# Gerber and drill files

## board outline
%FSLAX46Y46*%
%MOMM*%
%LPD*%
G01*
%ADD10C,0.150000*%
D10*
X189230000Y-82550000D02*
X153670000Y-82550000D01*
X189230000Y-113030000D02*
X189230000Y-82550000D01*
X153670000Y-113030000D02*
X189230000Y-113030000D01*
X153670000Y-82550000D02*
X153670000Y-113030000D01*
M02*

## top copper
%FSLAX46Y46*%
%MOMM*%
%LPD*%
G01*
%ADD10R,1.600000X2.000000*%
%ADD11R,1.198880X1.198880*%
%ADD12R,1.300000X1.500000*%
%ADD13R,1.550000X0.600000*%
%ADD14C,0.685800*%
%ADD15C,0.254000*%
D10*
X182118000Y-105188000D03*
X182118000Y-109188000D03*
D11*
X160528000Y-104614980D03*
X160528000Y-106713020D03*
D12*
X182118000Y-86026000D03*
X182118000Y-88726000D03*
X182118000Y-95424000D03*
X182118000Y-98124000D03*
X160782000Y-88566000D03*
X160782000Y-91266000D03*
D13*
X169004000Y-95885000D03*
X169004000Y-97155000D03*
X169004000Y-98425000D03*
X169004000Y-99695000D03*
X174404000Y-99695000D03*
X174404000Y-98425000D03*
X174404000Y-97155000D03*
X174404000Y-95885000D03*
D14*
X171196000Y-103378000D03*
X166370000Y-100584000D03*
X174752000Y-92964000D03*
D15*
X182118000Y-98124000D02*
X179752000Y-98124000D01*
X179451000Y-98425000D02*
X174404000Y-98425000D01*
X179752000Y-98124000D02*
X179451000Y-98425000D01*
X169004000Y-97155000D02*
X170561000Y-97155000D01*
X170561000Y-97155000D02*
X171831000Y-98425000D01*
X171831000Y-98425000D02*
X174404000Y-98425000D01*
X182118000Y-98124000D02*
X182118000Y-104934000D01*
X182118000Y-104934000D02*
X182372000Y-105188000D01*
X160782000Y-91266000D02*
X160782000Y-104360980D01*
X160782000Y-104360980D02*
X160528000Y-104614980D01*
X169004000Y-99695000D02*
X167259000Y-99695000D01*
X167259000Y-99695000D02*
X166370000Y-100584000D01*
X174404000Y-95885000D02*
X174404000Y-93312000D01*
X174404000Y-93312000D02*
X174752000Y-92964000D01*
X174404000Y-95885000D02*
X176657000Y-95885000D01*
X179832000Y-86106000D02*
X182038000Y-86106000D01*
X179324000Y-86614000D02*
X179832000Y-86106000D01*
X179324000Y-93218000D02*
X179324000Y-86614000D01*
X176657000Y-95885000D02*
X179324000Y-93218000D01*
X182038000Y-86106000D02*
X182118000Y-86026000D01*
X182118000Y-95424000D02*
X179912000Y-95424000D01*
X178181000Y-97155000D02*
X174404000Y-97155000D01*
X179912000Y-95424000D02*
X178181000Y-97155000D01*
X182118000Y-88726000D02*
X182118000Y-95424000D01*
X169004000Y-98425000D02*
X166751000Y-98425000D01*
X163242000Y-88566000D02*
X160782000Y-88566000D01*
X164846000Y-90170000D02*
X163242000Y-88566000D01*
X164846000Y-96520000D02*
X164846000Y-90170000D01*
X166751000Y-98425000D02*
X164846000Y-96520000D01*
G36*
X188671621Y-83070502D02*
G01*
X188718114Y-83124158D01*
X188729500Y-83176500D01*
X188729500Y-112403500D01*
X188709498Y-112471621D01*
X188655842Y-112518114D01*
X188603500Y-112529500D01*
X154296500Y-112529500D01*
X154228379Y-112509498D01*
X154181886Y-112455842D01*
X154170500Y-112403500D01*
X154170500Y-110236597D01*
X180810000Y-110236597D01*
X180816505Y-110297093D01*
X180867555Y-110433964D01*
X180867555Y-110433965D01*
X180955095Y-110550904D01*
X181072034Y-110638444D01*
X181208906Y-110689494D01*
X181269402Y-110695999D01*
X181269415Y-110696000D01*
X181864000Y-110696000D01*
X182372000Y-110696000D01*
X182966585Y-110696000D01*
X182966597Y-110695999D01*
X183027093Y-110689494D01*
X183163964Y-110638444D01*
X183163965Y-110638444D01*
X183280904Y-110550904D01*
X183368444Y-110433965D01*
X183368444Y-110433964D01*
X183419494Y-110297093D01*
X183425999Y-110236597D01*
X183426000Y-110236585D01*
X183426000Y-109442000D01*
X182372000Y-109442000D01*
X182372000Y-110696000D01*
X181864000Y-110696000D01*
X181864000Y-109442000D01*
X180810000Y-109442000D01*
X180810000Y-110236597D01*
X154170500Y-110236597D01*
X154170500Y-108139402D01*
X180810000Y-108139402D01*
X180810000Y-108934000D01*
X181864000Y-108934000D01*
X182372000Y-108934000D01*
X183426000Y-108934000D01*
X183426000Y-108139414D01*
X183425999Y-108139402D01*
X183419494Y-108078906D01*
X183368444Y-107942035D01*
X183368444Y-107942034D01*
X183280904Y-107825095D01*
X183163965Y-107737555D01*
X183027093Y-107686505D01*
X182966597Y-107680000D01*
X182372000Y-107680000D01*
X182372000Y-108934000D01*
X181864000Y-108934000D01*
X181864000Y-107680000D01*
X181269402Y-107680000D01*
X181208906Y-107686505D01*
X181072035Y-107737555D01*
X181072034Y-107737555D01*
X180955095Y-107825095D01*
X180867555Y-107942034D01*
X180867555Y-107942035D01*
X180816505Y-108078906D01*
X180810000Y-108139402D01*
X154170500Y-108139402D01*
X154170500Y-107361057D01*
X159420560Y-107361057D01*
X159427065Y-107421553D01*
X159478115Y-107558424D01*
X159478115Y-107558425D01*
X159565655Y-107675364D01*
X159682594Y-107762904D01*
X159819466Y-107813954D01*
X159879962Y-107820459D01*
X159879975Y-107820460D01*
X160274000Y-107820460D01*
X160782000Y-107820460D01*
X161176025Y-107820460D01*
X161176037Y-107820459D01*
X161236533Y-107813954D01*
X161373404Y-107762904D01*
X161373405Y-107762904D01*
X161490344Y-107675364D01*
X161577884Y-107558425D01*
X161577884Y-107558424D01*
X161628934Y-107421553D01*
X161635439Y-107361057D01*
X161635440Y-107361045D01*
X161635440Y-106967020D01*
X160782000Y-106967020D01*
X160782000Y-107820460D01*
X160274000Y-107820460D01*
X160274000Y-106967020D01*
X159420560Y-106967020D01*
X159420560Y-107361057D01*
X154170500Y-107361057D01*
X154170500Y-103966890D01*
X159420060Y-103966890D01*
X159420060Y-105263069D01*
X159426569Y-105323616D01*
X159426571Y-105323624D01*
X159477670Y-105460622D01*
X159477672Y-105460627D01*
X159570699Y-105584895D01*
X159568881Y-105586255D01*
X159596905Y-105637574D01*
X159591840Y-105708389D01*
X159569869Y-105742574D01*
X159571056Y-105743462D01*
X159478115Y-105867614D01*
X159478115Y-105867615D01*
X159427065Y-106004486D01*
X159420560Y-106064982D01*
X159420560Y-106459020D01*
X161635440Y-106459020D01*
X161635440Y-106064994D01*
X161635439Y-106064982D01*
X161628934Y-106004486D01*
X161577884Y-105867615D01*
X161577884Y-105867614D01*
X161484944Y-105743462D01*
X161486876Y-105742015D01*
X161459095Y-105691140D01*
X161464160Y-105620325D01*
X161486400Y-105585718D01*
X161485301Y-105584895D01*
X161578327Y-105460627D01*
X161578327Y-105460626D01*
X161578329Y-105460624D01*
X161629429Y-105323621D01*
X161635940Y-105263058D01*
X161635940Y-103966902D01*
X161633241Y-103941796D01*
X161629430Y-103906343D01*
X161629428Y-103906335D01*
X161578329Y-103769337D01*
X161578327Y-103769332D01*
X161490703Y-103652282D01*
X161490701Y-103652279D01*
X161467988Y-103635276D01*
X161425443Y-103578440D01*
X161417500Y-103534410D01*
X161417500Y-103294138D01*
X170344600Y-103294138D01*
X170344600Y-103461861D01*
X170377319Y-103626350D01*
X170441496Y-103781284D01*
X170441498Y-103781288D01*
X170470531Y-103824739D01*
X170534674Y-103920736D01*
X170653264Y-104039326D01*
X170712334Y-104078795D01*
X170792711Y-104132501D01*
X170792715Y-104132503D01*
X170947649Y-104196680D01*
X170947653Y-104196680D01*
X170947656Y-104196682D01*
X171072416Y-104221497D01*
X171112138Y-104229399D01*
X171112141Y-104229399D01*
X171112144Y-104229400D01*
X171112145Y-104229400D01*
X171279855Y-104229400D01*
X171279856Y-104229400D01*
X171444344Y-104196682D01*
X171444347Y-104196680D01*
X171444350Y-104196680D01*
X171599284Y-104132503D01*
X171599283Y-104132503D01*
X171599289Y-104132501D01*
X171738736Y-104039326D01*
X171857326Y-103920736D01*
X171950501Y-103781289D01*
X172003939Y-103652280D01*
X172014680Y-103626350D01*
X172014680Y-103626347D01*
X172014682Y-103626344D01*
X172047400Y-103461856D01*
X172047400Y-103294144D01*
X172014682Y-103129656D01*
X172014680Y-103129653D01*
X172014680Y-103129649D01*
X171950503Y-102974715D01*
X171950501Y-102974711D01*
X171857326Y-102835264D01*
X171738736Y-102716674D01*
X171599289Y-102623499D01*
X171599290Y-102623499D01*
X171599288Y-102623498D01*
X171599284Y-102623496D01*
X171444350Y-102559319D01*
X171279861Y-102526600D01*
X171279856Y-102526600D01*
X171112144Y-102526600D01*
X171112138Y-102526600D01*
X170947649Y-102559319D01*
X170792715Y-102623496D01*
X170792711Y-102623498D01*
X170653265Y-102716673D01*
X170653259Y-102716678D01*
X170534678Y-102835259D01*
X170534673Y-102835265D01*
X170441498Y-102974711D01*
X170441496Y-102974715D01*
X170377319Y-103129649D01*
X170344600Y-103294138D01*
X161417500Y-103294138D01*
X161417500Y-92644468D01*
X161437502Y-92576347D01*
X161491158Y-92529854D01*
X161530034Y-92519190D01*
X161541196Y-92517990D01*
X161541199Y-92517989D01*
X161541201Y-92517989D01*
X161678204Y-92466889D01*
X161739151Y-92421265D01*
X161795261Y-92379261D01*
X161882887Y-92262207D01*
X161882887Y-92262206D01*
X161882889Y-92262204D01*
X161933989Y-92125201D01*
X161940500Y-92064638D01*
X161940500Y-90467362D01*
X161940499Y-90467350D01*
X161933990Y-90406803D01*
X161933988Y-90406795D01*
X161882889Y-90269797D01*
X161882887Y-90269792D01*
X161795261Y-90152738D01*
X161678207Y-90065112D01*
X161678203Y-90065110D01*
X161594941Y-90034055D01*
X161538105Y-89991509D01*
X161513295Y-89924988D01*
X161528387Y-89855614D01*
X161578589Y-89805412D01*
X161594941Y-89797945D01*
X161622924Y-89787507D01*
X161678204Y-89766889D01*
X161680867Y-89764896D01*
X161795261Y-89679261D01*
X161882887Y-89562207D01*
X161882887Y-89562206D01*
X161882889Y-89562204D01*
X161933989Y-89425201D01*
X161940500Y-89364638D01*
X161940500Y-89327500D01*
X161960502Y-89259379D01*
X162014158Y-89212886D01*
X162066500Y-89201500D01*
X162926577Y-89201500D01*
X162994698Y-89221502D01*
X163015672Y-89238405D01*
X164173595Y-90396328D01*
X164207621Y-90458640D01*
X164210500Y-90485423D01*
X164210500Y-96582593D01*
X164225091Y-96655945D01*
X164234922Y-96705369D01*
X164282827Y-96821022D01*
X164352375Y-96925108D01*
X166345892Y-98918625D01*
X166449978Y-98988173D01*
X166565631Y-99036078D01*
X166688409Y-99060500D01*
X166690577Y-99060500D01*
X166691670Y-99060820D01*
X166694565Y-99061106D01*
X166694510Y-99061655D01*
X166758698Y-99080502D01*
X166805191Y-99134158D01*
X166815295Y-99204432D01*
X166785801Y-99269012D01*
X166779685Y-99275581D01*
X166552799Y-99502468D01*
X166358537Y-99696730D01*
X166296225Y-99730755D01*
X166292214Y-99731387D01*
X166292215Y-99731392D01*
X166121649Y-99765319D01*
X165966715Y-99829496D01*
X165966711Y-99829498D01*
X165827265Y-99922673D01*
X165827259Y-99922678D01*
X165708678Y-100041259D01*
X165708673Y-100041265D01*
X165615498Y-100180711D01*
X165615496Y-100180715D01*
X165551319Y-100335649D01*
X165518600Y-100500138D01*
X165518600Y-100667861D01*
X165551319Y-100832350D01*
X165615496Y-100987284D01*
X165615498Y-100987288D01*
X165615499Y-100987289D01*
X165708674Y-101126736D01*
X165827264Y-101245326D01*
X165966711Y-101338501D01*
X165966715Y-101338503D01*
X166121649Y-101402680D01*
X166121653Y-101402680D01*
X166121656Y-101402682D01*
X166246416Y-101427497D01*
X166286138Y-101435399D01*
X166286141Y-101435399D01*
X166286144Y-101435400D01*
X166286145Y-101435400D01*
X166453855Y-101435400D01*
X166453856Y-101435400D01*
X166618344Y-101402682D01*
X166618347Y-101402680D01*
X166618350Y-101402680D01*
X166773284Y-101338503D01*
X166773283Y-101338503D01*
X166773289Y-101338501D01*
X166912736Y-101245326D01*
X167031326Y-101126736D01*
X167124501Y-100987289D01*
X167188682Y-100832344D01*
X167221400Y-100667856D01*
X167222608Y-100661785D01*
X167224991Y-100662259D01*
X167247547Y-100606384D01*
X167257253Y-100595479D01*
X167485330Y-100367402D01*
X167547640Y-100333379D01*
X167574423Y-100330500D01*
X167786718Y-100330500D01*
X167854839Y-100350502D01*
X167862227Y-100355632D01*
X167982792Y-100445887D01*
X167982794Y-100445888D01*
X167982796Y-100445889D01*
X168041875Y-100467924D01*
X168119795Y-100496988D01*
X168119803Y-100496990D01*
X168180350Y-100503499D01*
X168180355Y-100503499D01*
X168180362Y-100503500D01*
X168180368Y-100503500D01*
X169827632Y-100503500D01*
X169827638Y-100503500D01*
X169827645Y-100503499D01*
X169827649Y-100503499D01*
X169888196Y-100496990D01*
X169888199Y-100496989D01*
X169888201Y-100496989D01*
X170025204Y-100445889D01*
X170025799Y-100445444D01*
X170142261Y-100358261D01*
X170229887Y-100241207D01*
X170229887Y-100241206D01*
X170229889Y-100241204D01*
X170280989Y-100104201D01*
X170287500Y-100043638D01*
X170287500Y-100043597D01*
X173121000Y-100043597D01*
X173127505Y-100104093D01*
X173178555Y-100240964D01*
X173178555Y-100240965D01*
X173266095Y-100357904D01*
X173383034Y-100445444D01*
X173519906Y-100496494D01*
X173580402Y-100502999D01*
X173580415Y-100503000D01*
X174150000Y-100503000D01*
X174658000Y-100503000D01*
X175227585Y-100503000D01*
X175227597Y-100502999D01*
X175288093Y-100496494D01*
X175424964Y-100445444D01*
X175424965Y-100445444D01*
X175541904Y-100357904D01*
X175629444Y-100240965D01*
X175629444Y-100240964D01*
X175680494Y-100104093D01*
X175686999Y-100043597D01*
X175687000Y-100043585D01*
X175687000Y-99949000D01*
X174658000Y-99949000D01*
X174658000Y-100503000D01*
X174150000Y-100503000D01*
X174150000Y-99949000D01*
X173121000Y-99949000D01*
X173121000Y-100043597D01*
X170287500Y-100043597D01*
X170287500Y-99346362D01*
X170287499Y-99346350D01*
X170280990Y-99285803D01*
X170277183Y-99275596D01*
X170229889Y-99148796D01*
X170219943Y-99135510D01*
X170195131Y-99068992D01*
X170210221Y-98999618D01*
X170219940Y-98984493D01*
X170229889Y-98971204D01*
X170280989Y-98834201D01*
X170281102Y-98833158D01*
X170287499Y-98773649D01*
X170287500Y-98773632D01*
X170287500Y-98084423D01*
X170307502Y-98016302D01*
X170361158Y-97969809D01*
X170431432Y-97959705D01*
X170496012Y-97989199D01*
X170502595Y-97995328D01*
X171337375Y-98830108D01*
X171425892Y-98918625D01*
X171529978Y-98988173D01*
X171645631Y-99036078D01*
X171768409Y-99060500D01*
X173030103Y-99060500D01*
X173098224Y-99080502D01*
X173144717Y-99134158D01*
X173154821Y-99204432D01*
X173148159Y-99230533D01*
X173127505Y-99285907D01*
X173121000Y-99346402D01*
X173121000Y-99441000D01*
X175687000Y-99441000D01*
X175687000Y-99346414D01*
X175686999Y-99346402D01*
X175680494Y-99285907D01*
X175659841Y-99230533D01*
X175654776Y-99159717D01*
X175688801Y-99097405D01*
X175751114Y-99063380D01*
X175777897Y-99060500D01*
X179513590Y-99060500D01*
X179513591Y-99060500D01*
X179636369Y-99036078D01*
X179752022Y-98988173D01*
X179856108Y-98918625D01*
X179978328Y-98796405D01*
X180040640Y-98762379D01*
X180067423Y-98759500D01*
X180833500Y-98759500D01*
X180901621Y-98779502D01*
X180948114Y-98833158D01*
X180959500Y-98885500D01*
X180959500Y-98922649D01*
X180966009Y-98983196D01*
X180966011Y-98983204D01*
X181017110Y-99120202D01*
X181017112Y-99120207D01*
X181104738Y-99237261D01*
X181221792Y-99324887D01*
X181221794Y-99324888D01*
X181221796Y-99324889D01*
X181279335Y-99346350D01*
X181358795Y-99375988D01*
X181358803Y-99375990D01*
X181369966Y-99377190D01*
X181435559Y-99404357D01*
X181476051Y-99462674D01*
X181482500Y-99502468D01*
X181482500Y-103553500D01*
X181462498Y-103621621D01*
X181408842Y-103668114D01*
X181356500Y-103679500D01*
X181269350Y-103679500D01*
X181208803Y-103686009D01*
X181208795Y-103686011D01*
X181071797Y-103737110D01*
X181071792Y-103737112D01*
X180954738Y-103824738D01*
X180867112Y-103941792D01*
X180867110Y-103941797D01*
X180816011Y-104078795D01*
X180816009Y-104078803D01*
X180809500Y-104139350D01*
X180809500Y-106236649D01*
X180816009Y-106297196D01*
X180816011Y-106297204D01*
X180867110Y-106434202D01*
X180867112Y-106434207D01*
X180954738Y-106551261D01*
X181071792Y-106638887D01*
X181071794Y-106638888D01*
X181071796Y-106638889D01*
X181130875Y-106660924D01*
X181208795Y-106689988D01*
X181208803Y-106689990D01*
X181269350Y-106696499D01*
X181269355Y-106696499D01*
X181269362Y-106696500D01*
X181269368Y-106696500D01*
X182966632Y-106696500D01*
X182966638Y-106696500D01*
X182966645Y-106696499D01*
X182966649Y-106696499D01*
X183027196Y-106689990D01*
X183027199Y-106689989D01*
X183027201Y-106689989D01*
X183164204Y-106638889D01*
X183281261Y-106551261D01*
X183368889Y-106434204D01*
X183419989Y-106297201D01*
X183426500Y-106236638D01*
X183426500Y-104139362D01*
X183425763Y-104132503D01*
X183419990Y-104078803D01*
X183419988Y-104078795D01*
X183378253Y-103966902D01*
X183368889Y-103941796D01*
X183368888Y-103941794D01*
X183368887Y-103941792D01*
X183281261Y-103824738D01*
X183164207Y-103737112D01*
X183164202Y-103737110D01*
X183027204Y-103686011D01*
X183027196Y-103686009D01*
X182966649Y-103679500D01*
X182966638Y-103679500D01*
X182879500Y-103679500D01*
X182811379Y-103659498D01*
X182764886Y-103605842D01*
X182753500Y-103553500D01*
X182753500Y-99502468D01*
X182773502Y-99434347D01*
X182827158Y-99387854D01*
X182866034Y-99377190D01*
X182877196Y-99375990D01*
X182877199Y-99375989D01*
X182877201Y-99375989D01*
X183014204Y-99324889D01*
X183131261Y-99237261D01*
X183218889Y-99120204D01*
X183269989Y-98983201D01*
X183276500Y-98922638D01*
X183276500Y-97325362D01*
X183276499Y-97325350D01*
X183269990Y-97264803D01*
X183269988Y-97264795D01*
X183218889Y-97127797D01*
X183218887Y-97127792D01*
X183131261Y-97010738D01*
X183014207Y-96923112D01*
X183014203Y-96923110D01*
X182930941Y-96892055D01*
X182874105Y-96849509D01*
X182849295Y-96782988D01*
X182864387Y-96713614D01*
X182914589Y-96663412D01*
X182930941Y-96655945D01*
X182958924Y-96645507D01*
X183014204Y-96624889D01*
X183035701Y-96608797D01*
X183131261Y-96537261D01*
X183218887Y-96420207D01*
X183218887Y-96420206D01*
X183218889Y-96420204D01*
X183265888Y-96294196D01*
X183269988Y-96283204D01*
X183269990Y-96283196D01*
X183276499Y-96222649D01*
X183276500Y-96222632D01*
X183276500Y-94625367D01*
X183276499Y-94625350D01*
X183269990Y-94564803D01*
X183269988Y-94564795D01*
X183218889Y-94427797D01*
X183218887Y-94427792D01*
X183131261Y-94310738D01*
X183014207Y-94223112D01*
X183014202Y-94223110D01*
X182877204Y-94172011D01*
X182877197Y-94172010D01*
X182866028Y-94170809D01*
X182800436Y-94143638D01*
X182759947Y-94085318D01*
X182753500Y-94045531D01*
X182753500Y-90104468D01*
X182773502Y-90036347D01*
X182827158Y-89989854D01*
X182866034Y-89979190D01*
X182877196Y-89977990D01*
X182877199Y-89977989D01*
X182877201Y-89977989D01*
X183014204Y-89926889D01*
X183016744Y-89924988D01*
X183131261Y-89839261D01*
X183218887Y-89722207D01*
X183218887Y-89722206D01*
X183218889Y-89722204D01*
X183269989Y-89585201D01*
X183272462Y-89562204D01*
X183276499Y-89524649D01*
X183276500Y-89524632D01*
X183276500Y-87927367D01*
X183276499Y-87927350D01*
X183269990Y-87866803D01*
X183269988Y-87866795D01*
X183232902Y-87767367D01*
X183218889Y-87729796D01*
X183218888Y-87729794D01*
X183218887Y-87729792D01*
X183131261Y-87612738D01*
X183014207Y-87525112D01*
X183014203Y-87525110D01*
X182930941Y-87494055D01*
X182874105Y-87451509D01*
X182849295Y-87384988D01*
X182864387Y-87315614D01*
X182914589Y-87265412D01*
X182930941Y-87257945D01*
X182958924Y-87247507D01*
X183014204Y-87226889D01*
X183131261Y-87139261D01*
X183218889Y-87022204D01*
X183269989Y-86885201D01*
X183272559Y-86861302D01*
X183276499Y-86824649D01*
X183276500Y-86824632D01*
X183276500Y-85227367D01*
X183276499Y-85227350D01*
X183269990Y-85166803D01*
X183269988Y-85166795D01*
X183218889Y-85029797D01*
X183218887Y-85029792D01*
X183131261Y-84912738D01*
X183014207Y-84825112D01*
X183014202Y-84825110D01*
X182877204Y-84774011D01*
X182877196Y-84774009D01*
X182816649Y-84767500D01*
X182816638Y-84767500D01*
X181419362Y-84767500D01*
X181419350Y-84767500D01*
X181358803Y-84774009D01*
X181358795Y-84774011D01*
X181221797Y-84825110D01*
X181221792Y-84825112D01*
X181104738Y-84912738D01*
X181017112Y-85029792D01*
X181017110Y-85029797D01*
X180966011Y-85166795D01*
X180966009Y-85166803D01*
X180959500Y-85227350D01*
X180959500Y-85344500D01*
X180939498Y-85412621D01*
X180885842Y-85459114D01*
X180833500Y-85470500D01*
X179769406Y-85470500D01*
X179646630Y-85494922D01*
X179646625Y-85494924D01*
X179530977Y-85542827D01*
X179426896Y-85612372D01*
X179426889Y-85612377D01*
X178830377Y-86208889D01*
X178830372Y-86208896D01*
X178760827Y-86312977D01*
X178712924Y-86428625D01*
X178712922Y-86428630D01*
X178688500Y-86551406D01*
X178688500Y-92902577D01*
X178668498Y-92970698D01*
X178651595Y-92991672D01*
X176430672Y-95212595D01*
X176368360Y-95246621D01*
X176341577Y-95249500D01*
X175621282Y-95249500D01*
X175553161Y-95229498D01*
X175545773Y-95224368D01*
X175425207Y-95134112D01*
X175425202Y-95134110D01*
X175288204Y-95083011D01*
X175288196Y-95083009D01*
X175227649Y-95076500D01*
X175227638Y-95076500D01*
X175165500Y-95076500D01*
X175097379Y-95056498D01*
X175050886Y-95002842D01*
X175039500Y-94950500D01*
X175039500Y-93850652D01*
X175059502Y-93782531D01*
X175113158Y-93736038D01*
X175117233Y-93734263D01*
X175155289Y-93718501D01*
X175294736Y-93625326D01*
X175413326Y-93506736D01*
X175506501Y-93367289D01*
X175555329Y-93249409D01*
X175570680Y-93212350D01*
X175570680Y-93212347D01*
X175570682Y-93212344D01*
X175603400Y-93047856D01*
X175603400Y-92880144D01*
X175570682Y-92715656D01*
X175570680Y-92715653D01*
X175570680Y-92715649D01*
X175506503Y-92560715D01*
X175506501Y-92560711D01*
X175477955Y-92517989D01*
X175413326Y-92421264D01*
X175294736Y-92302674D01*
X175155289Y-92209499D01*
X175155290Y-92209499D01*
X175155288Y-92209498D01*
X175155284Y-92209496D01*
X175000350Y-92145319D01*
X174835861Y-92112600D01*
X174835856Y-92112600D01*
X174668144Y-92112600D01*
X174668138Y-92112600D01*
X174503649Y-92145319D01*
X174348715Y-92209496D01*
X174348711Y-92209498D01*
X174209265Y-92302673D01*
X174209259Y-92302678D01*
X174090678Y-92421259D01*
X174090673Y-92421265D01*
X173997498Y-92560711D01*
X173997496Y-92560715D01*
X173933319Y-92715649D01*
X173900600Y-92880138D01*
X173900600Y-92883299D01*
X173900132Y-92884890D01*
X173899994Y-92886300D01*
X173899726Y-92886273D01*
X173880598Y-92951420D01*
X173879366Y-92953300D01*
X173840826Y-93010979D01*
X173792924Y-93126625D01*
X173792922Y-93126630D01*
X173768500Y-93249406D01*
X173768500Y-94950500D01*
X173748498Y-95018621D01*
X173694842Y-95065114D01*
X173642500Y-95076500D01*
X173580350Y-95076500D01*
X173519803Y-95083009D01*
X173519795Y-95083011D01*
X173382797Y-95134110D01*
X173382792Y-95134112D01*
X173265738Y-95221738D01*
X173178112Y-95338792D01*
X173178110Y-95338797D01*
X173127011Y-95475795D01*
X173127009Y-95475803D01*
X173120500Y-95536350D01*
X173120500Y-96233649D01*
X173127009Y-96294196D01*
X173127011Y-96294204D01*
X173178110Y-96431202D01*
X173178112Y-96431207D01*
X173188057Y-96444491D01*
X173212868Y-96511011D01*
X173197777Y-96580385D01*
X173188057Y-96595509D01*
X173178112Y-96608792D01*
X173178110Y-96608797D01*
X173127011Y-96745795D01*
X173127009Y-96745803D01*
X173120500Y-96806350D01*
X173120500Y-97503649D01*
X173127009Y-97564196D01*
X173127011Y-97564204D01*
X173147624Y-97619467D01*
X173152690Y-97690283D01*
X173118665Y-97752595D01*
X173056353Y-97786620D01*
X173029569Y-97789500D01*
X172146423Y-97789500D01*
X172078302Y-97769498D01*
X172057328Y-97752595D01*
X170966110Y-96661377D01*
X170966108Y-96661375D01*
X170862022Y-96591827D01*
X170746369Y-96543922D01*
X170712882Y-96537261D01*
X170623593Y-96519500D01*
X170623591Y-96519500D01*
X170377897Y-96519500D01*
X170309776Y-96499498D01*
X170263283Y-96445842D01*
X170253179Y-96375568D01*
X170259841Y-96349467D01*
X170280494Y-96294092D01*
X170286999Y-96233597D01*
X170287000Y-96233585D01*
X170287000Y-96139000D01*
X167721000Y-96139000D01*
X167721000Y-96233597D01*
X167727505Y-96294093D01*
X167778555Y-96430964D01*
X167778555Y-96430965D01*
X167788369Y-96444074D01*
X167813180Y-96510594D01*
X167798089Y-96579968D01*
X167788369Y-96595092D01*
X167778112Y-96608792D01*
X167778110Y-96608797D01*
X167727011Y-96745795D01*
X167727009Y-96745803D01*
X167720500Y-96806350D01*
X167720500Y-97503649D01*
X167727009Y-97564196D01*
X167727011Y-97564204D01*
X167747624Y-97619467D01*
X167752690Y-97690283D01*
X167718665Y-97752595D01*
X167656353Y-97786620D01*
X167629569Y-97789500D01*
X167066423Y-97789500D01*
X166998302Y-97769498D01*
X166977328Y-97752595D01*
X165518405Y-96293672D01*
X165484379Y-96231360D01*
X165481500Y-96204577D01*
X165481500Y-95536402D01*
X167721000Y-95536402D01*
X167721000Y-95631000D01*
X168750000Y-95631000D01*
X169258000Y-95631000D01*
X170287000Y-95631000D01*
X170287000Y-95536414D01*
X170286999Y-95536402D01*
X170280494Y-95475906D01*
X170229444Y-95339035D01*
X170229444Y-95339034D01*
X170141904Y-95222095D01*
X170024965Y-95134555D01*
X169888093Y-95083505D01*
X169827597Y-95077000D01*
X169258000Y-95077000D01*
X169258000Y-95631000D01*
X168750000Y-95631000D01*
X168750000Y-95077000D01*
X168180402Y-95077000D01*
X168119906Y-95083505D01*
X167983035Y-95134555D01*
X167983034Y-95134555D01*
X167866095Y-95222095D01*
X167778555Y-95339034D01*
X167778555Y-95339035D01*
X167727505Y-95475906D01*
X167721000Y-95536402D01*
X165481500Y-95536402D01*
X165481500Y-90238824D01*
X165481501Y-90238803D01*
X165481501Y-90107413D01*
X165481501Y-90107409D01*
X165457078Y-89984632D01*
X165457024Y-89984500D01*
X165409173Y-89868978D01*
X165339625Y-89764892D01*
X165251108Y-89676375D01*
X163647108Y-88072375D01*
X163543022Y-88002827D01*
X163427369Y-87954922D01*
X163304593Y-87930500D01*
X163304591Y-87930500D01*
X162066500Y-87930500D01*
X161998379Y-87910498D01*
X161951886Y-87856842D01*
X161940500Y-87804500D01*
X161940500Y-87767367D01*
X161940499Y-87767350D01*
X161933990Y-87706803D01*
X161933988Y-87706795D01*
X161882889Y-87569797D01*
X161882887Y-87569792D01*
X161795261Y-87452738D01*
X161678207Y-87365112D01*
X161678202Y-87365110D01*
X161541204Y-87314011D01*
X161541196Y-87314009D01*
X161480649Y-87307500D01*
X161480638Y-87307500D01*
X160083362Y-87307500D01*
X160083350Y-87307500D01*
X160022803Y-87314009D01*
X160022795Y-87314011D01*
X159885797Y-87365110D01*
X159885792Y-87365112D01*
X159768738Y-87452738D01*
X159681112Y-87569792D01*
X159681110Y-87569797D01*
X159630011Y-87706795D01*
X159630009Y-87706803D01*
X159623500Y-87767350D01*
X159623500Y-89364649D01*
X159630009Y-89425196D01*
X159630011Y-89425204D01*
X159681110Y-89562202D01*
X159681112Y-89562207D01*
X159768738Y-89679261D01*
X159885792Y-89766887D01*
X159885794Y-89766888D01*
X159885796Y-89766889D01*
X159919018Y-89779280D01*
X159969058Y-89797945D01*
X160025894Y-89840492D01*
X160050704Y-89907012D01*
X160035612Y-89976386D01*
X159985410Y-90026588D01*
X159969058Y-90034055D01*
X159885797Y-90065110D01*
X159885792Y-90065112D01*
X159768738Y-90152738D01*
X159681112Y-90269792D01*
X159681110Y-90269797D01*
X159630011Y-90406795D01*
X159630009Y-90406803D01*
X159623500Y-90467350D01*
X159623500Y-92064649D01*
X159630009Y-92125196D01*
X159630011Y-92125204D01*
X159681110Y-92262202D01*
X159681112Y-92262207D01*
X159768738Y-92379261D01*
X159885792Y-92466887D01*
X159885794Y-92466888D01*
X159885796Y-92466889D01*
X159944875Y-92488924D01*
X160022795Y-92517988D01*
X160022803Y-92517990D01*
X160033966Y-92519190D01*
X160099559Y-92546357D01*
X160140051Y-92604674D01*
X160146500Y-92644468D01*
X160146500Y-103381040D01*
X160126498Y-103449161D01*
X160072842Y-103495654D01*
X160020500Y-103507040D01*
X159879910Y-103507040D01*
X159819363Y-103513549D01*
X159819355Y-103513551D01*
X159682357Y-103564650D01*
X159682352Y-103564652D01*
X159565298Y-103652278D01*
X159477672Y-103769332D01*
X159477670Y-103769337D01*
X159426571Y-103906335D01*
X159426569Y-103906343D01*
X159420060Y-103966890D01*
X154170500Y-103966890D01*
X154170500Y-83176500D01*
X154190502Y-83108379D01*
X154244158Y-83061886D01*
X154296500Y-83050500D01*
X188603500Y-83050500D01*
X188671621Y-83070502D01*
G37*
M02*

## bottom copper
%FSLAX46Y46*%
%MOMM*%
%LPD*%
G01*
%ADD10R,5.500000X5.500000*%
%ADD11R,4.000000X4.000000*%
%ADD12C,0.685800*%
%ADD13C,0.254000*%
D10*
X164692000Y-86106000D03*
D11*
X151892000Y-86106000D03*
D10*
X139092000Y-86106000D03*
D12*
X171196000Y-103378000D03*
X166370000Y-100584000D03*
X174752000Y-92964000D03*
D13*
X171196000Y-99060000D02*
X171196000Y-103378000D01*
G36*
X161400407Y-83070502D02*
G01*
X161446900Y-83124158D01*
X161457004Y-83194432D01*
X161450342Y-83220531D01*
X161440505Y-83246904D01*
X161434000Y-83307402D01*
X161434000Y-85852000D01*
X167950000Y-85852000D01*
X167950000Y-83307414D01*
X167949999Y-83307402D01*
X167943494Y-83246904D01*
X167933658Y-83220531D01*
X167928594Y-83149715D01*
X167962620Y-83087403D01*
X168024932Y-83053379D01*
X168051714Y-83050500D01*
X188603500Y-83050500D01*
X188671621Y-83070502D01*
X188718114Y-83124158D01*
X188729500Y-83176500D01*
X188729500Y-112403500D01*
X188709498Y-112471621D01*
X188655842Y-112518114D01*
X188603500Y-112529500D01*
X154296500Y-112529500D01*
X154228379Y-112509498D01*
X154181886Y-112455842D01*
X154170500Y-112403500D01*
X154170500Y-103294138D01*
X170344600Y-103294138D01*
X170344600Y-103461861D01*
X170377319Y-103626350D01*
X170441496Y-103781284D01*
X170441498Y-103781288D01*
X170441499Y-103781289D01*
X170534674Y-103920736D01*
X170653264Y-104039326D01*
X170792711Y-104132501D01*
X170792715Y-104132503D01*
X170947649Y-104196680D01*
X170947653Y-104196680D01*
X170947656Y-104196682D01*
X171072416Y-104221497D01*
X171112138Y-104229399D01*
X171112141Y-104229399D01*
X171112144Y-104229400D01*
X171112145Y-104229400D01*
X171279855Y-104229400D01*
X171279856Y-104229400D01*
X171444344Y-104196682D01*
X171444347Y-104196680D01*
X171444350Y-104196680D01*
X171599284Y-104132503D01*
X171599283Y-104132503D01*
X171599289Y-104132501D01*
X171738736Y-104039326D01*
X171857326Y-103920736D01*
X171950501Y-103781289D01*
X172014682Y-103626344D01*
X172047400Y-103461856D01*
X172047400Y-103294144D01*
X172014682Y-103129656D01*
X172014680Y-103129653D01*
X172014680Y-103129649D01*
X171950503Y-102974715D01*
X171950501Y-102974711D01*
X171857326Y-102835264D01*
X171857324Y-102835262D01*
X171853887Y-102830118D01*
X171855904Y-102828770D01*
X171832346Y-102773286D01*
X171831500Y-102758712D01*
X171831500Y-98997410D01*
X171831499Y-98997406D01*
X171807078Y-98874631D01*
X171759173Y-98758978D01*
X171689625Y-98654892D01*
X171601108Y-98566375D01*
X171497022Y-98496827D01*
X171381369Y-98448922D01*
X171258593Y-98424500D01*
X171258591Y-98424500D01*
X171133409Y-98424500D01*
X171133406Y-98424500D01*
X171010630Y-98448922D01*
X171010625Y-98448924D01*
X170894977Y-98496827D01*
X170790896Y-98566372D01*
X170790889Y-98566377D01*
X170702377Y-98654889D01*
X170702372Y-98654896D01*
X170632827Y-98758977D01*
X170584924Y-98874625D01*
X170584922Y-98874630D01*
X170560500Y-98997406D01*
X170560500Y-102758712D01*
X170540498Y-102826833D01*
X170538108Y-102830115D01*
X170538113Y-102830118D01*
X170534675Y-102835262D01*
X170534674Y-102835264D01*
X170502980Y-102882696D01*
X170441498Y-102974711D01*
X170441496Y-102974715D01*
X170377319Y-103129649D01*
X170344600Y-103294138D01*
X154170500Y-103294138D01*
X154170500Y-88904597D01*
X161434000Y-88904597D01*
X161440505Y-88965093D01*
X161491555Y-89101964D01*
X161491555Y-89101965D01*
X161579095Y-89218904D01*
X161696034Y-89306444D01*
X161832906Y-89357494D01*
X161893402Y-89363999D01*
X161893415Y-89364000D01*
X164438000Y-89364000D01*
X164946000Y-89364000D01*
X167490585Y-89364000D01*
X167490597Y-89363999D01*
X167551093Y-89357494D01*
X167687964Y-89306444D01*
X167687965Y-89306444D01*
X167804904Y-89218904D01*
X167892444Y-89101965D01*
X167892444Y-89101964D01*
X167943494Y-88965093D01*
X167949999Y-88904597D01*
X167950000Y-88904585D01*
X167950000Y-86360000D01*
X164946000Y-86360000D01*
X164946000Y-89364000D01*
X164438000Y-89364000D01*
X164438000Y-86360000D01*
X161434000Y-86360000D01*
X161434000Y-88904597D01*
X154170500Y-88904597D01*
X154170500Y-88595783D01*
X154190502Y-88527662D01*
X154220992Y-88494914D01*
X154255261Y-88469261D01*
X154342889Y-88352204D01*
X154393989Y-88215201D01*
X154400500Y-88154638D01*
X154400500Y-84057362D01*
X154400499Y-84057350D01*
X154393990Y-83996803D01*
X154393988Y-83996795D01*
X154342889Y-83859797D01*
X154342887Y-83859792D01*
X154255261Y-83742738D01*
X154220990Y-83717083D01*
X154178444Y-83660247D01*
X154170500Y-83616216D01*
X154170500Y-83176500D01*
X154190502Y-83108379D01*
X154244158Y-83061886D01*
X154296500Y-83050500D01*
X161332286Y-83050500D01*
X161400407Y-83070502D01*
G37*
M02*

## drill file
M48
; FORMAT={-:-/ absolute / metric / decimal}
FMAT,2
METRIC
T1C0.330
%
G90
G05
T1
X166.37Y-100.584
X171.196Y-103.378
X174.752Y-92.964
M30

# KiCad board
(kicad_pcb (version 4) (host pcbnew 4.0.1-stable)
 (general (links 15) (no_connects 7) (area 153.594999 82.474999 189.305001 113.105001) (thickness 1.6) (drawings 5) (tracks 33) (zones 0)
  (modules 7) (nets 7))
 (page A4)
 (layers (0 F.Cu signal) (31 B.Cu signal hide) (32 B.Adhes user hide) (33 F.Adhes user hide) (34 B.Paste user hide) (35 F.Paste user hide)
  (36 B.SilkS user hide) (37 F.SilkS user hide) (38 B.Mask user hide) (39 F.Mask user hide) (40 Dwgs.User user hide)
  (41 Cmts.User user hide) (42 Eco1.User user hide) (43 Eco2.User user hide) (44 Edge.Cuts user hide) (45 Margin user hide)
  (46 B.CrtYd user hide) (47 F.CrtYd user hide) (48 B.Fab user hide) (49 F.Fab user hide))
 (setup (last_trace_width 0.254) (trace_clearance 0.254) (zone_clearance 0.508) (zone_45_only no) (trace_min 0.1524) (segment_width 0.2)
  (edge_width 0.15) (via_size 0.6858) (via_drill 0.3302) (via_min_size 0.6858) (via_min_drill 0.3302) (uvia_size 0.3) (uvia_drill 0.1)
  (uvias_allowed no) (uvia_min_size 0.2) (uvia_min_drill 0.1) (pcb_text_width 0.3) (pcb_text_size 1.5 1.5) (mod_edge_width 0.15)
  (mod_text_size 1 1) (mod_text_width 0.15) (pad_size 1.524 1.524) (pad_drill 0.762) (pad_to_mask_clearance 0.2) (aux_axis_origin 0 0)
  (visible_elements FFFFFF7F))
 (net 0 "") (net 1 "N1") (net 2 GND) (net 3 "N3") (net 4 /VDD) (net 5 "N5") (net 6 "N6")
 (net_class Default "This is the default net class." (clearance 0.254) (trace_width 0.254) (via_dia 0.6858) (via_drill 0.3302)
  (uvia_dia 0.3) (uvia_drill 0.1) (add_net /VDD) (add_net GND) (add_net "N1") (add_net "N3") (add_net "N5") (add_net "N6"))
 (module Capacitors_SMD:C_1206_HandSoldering (layer F.Cu) (at 182.118 107.188 270)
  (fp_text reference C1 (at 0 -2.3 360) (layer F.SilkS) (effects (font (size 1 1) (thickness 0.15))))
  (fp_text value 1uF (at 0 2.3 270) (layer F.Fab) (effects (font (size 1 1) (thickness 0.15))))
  (pad 1 smd rect (at -2 0 270) (size 2 1.6) (layers F.Cu F.Paste F.Mask) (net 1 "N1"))
  (pad 2 smd rect (at 2 0 270) (size 2 1.6) (layers F.Cu F.Paste F.Mask) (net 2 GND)))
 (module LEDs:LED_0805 (layer F.Cu) (at 160.528 105.664 90)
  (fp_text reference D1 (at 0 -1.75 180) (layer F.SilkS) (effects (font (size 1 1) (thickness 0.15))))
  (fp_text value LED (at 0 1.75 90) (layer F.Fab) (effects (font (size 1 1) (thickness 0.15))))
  (pad 2 smd rect (at 1.04902 0 270) (size 1.19888 1.19888) (layers F.Cu F.Paste F.Mask) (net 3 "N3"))
  (pad 1 smd rect (at -1.04902 0 270) (size 1.19888 1.19888) (layers F.Cu F.Paste F.Mask) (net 2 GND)))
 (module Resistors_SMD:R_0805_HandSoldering (layer F.Cu) (at 182.118 87.376 270)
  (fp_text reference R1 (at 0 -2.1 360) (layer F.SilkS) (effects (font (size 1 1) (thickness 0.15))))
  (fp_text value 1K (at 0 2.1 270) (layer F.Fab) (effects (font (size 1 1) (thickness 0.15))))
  (pad 1 smd rect (at -1.35 0 270) (size 1.5 1.3) (layers F.Cu F.Paste F.Mask) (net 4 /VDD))
  (pad 2 smd rect (at 1.35 0 270) (size 1.5 1.3) (layers F.Cu F.Paste F.Mask) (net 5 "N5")))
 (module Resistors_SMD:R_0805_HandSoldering (layer F.Cu) (at 182.118 96.774 270)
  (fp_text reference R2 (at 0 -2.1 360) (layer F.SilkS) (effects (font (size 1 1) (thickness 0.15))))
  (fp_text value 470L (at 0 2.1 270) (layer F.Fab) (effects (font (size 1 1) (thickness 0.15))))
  (pad 1 smd rect (at -1.35 0 270) (size 1.5 1.3) (layers F.Cu F.Paste F.Mask) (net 5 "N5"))
  (pad 2 smd rect (at 1.35 0 270) (size 1.5 1.3) (layers F.Cu F.Paste F.Mask) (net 1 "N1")))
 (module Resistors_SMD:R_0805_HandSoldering (layer F.Cu) (at 160.782 89.916 270)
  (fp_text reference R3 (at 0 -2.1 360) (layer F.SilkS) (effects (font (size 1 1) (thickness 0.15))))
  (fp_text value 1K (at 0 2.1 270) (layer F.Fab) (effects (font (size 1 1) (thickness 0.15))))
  (pad 1 smd rect (at -1.35 0 270) (size 1.5 1.3) (layers F.Cu F.Paste F.Mask) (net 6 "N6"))
  (pad 2 smd rect (at 1.35 0 270) (size 1.5 1.3) (layers F.Cu F.Paste F.Mask) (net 3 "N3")))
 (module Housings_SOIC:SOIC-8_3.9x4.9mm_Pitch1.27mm (layer F.Cu) (at 171.704 97.79)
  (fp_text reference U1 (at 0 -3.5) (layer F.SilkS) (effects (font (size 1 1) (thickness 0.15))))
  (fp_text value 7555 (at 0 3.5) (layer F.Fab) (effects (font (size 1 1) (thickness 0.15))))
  (pad 1 smd rect (at -2.7 -1.905) (size 1.55 0.6) (layers F.Cu F.Paste F.Mask) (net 2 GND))
  (pad 2 smd rect (at -2.7 -0.635) (size 1.55 0.6) (layers F.Cu F.Paste F.Mask) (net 1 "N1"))
  (pad 3 smd rect (at -2.7 0.635) (size 1.55 0.6) (layers F.Cu F.Paste F.Mask) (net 6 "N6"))
  (pad 4 smd rect (at -2.7 1.905) (size 1.55 0.6) (layers F.Cu F.Paste F.Mask) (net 4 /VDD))
  (pad 5 smd rect (at 2.7 1.905) (size 1.55 0.6) (layers F.Cu F.Paste F.Mask) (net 2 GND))
  (pad 6 smd rect (at 2.7 0.635) (size 1.55 0.6) (layers F.Cu F.Paste F.Mask) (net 1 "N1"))
  (pad 7 smd rect (at 2.7 -0.635) (size 1.55 0.6) (layers F.Cu F.Paste F.Mask) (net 5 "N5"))
  (pad 8 smd rect (at 2.7 -1.905) (size 1.55 0.6) (layers F.Cu F.Paste F.Mask) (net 4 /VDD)))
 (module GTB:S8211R (layer B.Cu) (at 151.892 86.106)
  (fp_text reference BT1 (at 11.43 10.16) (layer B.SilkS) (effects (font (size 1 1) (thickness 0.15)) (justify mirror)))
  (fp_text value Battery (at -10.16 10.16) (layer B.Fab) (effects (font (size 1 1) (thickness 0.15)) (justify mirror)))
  (pad 1 smd rect (at 12.8 0) (size 5.5 5.5) (layers B.Cu B.Paste B.Mask) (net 4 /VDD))
  (pad 2 smd rect (at 0 0) (size 4 4) (layers B.Cu B.Paste B.Mask) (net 2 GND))
  (pad 1 smd rect (at -12.8 0) (size 5.5 5.5) (layers B.Cu B.Paste B.Mask) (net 4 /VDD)))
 (gr_line (start 189.23 82.55) (end 153.67 82.55) (angle 90) (layer Edge.Cuts) (width 0.15))
 (gr_line (start 189.23 113.03) (end 189.23 82.55) (angle 90) (layer Edge.Cuts) (width 0.15))
 (gr_line (start 153.67 113.03) (end 189.23 113.03) (angle 90) (layer Edge.Cuts) (width 0.15))
 (gr_line (start 153.67 82.55) (end 153.67 113.03) (angle 90) (layer Edge.Cuts) (width 0.15))
 (segment (start 171.196 99.06) (end 171.196 103.378) (width 0.254) (layer B.Cu) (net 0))
 (via (at 171.196 103.378) (size 0.6858) (drill 0.3302) (layers F.Cu B.Cu) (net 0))
 (segment (start 182.118 98.124) (end 179.752 98.124) (width 0.254) (layer F.Cu) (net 1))
 (segment (start 179.451 98.425) (end 174.404 98.425) (width 0.254) (layer F.Cu) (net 1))
 (segment (start 179.752 98.124) (end 179.451 98.425) (width 0.254) (layer F.Cu) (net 1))
 (segment (start 169.004 97.155) (end 170.561 97.155) (width 0.254) (layer F.Cu) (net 1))
 (segment (start 170.561 97.155) (end 171.831 98.425) (width 0.254) (layer F.Cu) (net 1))
 (segment (start 171.831 98.425) (end 174.404 98.425) (width 0.254) (layer F.Cu) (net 1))
 (segment (start 182.118 98.124) (end 182.118 104.934) (width 0.254) (layer F.Cu) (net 1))
 (segment (start 182.118 104.934) (end 182.372 105.188) (width 0.254) (layer F.Cu) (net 1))
 (segment (start 160.782 91.266) (end 160.782 104.36098) (width 0.254) (layer F.Cu) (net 3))
 (segment (start 160.782 104.36098) (end 160.528 104.61498) (width 0.254) (layer F.Cu) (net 3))
 (segment (start 169.004 99.695) (end 167.259 99.695) (width 0.254) (layer F.Cu) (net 4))
 (via (at 166.37 100.584) (size 0.6858) (drill 0.3302) (layers F.Cu B.Cu) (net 4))
 (segment (start 167.259 99.695) (end 166.37 100.584) (width 0.254) (layer F.Cu) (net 4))
 (segment (start 174.404 95.885) (end 174.404 93.312) (width 0.254) (layer F.Cu) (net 4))
 (via (at 174.752 92.964) (size 0.6858) (drill 0.3302) (layers F.Cu B.Cu) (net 4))
 (segment (start 174.404 93.312) (end 174.752 92.964) (width 0.254) (layer F.Cu) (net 4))
 (segment (start 174.404 95.885) (end 176.657 95.885) (width 0.254) (layer F.Cu) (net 4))
 (segment (start 179.832 86.106) (end 182.038 86.106) (width 0.254) (layer F.Cu) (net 4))
 (segment (start 179.324 86.614) (end 179.832 86.106) (width 0.254) (layer F.Cu) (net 4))
 (segment (start 179.324 93.218) (end 179.324 86.614) (width 0.254) (layer F.Cu) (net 4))
 (segment (start 176.657 95.885) (end 179.324 93.218) (width 0.254) (layer F.Cu) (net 4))
 (segment (start 182.038 86.106) (end 182.118 86.026) (width 0.254) (layer F.Cu) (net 4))
 (segment (start 182.118 95.424) (end 179.912 95.424) (width 0.254) (layer F.Cu) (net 5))
 (segment (start 178.181 97.155) (end 174.404 97.155) (width 0.254) (layer F.Cu) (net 5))
 (segment (start 179.912 95.424) (end 178.181 97.155) (width 0.254) (layer F.Cu) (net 5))
 (segment (start 182.118 88.726) (end 182.118 95.424) (width 0.254) (layer F.Cu) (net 5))
 (segment (start 169.004 98.425) (end 166.751 98.425) (width 0.254) (layer F.Cu) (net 6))
 (segment (start 163.242 88.566) (end 160.782 88.566) (width 0.254) (layer F.Cu) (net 6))
 (segment (start 164.846 90.17) (end 163.242 88.566) (width 0.254) (layer F.Cu) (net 6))
 (segment (start 164.846 96.52) (end 164.846 90.17) (width 0.254) (layer F.Cu) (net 6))
 (segment (start 166.751 98.425) (end 164.846 96.52) (width 0.254) (layer F.Cu) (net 6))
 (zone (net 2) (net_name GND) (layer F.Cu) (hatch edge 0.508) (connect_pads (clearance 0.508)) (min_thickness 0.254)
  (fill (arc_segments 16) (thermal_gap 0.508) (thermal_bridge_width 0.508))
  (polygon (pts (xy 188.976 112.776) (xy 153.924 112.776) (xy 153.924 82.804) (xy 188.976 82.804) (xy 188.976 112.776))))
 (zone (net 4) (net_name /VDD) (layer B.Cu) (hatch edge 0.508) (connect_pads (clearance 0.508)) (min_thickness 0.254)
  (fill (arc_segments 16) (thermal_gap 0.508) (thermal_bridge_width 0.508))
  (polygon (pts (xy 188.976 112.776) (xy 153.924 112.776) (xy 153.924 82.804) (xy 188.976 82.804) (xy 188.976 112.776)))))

